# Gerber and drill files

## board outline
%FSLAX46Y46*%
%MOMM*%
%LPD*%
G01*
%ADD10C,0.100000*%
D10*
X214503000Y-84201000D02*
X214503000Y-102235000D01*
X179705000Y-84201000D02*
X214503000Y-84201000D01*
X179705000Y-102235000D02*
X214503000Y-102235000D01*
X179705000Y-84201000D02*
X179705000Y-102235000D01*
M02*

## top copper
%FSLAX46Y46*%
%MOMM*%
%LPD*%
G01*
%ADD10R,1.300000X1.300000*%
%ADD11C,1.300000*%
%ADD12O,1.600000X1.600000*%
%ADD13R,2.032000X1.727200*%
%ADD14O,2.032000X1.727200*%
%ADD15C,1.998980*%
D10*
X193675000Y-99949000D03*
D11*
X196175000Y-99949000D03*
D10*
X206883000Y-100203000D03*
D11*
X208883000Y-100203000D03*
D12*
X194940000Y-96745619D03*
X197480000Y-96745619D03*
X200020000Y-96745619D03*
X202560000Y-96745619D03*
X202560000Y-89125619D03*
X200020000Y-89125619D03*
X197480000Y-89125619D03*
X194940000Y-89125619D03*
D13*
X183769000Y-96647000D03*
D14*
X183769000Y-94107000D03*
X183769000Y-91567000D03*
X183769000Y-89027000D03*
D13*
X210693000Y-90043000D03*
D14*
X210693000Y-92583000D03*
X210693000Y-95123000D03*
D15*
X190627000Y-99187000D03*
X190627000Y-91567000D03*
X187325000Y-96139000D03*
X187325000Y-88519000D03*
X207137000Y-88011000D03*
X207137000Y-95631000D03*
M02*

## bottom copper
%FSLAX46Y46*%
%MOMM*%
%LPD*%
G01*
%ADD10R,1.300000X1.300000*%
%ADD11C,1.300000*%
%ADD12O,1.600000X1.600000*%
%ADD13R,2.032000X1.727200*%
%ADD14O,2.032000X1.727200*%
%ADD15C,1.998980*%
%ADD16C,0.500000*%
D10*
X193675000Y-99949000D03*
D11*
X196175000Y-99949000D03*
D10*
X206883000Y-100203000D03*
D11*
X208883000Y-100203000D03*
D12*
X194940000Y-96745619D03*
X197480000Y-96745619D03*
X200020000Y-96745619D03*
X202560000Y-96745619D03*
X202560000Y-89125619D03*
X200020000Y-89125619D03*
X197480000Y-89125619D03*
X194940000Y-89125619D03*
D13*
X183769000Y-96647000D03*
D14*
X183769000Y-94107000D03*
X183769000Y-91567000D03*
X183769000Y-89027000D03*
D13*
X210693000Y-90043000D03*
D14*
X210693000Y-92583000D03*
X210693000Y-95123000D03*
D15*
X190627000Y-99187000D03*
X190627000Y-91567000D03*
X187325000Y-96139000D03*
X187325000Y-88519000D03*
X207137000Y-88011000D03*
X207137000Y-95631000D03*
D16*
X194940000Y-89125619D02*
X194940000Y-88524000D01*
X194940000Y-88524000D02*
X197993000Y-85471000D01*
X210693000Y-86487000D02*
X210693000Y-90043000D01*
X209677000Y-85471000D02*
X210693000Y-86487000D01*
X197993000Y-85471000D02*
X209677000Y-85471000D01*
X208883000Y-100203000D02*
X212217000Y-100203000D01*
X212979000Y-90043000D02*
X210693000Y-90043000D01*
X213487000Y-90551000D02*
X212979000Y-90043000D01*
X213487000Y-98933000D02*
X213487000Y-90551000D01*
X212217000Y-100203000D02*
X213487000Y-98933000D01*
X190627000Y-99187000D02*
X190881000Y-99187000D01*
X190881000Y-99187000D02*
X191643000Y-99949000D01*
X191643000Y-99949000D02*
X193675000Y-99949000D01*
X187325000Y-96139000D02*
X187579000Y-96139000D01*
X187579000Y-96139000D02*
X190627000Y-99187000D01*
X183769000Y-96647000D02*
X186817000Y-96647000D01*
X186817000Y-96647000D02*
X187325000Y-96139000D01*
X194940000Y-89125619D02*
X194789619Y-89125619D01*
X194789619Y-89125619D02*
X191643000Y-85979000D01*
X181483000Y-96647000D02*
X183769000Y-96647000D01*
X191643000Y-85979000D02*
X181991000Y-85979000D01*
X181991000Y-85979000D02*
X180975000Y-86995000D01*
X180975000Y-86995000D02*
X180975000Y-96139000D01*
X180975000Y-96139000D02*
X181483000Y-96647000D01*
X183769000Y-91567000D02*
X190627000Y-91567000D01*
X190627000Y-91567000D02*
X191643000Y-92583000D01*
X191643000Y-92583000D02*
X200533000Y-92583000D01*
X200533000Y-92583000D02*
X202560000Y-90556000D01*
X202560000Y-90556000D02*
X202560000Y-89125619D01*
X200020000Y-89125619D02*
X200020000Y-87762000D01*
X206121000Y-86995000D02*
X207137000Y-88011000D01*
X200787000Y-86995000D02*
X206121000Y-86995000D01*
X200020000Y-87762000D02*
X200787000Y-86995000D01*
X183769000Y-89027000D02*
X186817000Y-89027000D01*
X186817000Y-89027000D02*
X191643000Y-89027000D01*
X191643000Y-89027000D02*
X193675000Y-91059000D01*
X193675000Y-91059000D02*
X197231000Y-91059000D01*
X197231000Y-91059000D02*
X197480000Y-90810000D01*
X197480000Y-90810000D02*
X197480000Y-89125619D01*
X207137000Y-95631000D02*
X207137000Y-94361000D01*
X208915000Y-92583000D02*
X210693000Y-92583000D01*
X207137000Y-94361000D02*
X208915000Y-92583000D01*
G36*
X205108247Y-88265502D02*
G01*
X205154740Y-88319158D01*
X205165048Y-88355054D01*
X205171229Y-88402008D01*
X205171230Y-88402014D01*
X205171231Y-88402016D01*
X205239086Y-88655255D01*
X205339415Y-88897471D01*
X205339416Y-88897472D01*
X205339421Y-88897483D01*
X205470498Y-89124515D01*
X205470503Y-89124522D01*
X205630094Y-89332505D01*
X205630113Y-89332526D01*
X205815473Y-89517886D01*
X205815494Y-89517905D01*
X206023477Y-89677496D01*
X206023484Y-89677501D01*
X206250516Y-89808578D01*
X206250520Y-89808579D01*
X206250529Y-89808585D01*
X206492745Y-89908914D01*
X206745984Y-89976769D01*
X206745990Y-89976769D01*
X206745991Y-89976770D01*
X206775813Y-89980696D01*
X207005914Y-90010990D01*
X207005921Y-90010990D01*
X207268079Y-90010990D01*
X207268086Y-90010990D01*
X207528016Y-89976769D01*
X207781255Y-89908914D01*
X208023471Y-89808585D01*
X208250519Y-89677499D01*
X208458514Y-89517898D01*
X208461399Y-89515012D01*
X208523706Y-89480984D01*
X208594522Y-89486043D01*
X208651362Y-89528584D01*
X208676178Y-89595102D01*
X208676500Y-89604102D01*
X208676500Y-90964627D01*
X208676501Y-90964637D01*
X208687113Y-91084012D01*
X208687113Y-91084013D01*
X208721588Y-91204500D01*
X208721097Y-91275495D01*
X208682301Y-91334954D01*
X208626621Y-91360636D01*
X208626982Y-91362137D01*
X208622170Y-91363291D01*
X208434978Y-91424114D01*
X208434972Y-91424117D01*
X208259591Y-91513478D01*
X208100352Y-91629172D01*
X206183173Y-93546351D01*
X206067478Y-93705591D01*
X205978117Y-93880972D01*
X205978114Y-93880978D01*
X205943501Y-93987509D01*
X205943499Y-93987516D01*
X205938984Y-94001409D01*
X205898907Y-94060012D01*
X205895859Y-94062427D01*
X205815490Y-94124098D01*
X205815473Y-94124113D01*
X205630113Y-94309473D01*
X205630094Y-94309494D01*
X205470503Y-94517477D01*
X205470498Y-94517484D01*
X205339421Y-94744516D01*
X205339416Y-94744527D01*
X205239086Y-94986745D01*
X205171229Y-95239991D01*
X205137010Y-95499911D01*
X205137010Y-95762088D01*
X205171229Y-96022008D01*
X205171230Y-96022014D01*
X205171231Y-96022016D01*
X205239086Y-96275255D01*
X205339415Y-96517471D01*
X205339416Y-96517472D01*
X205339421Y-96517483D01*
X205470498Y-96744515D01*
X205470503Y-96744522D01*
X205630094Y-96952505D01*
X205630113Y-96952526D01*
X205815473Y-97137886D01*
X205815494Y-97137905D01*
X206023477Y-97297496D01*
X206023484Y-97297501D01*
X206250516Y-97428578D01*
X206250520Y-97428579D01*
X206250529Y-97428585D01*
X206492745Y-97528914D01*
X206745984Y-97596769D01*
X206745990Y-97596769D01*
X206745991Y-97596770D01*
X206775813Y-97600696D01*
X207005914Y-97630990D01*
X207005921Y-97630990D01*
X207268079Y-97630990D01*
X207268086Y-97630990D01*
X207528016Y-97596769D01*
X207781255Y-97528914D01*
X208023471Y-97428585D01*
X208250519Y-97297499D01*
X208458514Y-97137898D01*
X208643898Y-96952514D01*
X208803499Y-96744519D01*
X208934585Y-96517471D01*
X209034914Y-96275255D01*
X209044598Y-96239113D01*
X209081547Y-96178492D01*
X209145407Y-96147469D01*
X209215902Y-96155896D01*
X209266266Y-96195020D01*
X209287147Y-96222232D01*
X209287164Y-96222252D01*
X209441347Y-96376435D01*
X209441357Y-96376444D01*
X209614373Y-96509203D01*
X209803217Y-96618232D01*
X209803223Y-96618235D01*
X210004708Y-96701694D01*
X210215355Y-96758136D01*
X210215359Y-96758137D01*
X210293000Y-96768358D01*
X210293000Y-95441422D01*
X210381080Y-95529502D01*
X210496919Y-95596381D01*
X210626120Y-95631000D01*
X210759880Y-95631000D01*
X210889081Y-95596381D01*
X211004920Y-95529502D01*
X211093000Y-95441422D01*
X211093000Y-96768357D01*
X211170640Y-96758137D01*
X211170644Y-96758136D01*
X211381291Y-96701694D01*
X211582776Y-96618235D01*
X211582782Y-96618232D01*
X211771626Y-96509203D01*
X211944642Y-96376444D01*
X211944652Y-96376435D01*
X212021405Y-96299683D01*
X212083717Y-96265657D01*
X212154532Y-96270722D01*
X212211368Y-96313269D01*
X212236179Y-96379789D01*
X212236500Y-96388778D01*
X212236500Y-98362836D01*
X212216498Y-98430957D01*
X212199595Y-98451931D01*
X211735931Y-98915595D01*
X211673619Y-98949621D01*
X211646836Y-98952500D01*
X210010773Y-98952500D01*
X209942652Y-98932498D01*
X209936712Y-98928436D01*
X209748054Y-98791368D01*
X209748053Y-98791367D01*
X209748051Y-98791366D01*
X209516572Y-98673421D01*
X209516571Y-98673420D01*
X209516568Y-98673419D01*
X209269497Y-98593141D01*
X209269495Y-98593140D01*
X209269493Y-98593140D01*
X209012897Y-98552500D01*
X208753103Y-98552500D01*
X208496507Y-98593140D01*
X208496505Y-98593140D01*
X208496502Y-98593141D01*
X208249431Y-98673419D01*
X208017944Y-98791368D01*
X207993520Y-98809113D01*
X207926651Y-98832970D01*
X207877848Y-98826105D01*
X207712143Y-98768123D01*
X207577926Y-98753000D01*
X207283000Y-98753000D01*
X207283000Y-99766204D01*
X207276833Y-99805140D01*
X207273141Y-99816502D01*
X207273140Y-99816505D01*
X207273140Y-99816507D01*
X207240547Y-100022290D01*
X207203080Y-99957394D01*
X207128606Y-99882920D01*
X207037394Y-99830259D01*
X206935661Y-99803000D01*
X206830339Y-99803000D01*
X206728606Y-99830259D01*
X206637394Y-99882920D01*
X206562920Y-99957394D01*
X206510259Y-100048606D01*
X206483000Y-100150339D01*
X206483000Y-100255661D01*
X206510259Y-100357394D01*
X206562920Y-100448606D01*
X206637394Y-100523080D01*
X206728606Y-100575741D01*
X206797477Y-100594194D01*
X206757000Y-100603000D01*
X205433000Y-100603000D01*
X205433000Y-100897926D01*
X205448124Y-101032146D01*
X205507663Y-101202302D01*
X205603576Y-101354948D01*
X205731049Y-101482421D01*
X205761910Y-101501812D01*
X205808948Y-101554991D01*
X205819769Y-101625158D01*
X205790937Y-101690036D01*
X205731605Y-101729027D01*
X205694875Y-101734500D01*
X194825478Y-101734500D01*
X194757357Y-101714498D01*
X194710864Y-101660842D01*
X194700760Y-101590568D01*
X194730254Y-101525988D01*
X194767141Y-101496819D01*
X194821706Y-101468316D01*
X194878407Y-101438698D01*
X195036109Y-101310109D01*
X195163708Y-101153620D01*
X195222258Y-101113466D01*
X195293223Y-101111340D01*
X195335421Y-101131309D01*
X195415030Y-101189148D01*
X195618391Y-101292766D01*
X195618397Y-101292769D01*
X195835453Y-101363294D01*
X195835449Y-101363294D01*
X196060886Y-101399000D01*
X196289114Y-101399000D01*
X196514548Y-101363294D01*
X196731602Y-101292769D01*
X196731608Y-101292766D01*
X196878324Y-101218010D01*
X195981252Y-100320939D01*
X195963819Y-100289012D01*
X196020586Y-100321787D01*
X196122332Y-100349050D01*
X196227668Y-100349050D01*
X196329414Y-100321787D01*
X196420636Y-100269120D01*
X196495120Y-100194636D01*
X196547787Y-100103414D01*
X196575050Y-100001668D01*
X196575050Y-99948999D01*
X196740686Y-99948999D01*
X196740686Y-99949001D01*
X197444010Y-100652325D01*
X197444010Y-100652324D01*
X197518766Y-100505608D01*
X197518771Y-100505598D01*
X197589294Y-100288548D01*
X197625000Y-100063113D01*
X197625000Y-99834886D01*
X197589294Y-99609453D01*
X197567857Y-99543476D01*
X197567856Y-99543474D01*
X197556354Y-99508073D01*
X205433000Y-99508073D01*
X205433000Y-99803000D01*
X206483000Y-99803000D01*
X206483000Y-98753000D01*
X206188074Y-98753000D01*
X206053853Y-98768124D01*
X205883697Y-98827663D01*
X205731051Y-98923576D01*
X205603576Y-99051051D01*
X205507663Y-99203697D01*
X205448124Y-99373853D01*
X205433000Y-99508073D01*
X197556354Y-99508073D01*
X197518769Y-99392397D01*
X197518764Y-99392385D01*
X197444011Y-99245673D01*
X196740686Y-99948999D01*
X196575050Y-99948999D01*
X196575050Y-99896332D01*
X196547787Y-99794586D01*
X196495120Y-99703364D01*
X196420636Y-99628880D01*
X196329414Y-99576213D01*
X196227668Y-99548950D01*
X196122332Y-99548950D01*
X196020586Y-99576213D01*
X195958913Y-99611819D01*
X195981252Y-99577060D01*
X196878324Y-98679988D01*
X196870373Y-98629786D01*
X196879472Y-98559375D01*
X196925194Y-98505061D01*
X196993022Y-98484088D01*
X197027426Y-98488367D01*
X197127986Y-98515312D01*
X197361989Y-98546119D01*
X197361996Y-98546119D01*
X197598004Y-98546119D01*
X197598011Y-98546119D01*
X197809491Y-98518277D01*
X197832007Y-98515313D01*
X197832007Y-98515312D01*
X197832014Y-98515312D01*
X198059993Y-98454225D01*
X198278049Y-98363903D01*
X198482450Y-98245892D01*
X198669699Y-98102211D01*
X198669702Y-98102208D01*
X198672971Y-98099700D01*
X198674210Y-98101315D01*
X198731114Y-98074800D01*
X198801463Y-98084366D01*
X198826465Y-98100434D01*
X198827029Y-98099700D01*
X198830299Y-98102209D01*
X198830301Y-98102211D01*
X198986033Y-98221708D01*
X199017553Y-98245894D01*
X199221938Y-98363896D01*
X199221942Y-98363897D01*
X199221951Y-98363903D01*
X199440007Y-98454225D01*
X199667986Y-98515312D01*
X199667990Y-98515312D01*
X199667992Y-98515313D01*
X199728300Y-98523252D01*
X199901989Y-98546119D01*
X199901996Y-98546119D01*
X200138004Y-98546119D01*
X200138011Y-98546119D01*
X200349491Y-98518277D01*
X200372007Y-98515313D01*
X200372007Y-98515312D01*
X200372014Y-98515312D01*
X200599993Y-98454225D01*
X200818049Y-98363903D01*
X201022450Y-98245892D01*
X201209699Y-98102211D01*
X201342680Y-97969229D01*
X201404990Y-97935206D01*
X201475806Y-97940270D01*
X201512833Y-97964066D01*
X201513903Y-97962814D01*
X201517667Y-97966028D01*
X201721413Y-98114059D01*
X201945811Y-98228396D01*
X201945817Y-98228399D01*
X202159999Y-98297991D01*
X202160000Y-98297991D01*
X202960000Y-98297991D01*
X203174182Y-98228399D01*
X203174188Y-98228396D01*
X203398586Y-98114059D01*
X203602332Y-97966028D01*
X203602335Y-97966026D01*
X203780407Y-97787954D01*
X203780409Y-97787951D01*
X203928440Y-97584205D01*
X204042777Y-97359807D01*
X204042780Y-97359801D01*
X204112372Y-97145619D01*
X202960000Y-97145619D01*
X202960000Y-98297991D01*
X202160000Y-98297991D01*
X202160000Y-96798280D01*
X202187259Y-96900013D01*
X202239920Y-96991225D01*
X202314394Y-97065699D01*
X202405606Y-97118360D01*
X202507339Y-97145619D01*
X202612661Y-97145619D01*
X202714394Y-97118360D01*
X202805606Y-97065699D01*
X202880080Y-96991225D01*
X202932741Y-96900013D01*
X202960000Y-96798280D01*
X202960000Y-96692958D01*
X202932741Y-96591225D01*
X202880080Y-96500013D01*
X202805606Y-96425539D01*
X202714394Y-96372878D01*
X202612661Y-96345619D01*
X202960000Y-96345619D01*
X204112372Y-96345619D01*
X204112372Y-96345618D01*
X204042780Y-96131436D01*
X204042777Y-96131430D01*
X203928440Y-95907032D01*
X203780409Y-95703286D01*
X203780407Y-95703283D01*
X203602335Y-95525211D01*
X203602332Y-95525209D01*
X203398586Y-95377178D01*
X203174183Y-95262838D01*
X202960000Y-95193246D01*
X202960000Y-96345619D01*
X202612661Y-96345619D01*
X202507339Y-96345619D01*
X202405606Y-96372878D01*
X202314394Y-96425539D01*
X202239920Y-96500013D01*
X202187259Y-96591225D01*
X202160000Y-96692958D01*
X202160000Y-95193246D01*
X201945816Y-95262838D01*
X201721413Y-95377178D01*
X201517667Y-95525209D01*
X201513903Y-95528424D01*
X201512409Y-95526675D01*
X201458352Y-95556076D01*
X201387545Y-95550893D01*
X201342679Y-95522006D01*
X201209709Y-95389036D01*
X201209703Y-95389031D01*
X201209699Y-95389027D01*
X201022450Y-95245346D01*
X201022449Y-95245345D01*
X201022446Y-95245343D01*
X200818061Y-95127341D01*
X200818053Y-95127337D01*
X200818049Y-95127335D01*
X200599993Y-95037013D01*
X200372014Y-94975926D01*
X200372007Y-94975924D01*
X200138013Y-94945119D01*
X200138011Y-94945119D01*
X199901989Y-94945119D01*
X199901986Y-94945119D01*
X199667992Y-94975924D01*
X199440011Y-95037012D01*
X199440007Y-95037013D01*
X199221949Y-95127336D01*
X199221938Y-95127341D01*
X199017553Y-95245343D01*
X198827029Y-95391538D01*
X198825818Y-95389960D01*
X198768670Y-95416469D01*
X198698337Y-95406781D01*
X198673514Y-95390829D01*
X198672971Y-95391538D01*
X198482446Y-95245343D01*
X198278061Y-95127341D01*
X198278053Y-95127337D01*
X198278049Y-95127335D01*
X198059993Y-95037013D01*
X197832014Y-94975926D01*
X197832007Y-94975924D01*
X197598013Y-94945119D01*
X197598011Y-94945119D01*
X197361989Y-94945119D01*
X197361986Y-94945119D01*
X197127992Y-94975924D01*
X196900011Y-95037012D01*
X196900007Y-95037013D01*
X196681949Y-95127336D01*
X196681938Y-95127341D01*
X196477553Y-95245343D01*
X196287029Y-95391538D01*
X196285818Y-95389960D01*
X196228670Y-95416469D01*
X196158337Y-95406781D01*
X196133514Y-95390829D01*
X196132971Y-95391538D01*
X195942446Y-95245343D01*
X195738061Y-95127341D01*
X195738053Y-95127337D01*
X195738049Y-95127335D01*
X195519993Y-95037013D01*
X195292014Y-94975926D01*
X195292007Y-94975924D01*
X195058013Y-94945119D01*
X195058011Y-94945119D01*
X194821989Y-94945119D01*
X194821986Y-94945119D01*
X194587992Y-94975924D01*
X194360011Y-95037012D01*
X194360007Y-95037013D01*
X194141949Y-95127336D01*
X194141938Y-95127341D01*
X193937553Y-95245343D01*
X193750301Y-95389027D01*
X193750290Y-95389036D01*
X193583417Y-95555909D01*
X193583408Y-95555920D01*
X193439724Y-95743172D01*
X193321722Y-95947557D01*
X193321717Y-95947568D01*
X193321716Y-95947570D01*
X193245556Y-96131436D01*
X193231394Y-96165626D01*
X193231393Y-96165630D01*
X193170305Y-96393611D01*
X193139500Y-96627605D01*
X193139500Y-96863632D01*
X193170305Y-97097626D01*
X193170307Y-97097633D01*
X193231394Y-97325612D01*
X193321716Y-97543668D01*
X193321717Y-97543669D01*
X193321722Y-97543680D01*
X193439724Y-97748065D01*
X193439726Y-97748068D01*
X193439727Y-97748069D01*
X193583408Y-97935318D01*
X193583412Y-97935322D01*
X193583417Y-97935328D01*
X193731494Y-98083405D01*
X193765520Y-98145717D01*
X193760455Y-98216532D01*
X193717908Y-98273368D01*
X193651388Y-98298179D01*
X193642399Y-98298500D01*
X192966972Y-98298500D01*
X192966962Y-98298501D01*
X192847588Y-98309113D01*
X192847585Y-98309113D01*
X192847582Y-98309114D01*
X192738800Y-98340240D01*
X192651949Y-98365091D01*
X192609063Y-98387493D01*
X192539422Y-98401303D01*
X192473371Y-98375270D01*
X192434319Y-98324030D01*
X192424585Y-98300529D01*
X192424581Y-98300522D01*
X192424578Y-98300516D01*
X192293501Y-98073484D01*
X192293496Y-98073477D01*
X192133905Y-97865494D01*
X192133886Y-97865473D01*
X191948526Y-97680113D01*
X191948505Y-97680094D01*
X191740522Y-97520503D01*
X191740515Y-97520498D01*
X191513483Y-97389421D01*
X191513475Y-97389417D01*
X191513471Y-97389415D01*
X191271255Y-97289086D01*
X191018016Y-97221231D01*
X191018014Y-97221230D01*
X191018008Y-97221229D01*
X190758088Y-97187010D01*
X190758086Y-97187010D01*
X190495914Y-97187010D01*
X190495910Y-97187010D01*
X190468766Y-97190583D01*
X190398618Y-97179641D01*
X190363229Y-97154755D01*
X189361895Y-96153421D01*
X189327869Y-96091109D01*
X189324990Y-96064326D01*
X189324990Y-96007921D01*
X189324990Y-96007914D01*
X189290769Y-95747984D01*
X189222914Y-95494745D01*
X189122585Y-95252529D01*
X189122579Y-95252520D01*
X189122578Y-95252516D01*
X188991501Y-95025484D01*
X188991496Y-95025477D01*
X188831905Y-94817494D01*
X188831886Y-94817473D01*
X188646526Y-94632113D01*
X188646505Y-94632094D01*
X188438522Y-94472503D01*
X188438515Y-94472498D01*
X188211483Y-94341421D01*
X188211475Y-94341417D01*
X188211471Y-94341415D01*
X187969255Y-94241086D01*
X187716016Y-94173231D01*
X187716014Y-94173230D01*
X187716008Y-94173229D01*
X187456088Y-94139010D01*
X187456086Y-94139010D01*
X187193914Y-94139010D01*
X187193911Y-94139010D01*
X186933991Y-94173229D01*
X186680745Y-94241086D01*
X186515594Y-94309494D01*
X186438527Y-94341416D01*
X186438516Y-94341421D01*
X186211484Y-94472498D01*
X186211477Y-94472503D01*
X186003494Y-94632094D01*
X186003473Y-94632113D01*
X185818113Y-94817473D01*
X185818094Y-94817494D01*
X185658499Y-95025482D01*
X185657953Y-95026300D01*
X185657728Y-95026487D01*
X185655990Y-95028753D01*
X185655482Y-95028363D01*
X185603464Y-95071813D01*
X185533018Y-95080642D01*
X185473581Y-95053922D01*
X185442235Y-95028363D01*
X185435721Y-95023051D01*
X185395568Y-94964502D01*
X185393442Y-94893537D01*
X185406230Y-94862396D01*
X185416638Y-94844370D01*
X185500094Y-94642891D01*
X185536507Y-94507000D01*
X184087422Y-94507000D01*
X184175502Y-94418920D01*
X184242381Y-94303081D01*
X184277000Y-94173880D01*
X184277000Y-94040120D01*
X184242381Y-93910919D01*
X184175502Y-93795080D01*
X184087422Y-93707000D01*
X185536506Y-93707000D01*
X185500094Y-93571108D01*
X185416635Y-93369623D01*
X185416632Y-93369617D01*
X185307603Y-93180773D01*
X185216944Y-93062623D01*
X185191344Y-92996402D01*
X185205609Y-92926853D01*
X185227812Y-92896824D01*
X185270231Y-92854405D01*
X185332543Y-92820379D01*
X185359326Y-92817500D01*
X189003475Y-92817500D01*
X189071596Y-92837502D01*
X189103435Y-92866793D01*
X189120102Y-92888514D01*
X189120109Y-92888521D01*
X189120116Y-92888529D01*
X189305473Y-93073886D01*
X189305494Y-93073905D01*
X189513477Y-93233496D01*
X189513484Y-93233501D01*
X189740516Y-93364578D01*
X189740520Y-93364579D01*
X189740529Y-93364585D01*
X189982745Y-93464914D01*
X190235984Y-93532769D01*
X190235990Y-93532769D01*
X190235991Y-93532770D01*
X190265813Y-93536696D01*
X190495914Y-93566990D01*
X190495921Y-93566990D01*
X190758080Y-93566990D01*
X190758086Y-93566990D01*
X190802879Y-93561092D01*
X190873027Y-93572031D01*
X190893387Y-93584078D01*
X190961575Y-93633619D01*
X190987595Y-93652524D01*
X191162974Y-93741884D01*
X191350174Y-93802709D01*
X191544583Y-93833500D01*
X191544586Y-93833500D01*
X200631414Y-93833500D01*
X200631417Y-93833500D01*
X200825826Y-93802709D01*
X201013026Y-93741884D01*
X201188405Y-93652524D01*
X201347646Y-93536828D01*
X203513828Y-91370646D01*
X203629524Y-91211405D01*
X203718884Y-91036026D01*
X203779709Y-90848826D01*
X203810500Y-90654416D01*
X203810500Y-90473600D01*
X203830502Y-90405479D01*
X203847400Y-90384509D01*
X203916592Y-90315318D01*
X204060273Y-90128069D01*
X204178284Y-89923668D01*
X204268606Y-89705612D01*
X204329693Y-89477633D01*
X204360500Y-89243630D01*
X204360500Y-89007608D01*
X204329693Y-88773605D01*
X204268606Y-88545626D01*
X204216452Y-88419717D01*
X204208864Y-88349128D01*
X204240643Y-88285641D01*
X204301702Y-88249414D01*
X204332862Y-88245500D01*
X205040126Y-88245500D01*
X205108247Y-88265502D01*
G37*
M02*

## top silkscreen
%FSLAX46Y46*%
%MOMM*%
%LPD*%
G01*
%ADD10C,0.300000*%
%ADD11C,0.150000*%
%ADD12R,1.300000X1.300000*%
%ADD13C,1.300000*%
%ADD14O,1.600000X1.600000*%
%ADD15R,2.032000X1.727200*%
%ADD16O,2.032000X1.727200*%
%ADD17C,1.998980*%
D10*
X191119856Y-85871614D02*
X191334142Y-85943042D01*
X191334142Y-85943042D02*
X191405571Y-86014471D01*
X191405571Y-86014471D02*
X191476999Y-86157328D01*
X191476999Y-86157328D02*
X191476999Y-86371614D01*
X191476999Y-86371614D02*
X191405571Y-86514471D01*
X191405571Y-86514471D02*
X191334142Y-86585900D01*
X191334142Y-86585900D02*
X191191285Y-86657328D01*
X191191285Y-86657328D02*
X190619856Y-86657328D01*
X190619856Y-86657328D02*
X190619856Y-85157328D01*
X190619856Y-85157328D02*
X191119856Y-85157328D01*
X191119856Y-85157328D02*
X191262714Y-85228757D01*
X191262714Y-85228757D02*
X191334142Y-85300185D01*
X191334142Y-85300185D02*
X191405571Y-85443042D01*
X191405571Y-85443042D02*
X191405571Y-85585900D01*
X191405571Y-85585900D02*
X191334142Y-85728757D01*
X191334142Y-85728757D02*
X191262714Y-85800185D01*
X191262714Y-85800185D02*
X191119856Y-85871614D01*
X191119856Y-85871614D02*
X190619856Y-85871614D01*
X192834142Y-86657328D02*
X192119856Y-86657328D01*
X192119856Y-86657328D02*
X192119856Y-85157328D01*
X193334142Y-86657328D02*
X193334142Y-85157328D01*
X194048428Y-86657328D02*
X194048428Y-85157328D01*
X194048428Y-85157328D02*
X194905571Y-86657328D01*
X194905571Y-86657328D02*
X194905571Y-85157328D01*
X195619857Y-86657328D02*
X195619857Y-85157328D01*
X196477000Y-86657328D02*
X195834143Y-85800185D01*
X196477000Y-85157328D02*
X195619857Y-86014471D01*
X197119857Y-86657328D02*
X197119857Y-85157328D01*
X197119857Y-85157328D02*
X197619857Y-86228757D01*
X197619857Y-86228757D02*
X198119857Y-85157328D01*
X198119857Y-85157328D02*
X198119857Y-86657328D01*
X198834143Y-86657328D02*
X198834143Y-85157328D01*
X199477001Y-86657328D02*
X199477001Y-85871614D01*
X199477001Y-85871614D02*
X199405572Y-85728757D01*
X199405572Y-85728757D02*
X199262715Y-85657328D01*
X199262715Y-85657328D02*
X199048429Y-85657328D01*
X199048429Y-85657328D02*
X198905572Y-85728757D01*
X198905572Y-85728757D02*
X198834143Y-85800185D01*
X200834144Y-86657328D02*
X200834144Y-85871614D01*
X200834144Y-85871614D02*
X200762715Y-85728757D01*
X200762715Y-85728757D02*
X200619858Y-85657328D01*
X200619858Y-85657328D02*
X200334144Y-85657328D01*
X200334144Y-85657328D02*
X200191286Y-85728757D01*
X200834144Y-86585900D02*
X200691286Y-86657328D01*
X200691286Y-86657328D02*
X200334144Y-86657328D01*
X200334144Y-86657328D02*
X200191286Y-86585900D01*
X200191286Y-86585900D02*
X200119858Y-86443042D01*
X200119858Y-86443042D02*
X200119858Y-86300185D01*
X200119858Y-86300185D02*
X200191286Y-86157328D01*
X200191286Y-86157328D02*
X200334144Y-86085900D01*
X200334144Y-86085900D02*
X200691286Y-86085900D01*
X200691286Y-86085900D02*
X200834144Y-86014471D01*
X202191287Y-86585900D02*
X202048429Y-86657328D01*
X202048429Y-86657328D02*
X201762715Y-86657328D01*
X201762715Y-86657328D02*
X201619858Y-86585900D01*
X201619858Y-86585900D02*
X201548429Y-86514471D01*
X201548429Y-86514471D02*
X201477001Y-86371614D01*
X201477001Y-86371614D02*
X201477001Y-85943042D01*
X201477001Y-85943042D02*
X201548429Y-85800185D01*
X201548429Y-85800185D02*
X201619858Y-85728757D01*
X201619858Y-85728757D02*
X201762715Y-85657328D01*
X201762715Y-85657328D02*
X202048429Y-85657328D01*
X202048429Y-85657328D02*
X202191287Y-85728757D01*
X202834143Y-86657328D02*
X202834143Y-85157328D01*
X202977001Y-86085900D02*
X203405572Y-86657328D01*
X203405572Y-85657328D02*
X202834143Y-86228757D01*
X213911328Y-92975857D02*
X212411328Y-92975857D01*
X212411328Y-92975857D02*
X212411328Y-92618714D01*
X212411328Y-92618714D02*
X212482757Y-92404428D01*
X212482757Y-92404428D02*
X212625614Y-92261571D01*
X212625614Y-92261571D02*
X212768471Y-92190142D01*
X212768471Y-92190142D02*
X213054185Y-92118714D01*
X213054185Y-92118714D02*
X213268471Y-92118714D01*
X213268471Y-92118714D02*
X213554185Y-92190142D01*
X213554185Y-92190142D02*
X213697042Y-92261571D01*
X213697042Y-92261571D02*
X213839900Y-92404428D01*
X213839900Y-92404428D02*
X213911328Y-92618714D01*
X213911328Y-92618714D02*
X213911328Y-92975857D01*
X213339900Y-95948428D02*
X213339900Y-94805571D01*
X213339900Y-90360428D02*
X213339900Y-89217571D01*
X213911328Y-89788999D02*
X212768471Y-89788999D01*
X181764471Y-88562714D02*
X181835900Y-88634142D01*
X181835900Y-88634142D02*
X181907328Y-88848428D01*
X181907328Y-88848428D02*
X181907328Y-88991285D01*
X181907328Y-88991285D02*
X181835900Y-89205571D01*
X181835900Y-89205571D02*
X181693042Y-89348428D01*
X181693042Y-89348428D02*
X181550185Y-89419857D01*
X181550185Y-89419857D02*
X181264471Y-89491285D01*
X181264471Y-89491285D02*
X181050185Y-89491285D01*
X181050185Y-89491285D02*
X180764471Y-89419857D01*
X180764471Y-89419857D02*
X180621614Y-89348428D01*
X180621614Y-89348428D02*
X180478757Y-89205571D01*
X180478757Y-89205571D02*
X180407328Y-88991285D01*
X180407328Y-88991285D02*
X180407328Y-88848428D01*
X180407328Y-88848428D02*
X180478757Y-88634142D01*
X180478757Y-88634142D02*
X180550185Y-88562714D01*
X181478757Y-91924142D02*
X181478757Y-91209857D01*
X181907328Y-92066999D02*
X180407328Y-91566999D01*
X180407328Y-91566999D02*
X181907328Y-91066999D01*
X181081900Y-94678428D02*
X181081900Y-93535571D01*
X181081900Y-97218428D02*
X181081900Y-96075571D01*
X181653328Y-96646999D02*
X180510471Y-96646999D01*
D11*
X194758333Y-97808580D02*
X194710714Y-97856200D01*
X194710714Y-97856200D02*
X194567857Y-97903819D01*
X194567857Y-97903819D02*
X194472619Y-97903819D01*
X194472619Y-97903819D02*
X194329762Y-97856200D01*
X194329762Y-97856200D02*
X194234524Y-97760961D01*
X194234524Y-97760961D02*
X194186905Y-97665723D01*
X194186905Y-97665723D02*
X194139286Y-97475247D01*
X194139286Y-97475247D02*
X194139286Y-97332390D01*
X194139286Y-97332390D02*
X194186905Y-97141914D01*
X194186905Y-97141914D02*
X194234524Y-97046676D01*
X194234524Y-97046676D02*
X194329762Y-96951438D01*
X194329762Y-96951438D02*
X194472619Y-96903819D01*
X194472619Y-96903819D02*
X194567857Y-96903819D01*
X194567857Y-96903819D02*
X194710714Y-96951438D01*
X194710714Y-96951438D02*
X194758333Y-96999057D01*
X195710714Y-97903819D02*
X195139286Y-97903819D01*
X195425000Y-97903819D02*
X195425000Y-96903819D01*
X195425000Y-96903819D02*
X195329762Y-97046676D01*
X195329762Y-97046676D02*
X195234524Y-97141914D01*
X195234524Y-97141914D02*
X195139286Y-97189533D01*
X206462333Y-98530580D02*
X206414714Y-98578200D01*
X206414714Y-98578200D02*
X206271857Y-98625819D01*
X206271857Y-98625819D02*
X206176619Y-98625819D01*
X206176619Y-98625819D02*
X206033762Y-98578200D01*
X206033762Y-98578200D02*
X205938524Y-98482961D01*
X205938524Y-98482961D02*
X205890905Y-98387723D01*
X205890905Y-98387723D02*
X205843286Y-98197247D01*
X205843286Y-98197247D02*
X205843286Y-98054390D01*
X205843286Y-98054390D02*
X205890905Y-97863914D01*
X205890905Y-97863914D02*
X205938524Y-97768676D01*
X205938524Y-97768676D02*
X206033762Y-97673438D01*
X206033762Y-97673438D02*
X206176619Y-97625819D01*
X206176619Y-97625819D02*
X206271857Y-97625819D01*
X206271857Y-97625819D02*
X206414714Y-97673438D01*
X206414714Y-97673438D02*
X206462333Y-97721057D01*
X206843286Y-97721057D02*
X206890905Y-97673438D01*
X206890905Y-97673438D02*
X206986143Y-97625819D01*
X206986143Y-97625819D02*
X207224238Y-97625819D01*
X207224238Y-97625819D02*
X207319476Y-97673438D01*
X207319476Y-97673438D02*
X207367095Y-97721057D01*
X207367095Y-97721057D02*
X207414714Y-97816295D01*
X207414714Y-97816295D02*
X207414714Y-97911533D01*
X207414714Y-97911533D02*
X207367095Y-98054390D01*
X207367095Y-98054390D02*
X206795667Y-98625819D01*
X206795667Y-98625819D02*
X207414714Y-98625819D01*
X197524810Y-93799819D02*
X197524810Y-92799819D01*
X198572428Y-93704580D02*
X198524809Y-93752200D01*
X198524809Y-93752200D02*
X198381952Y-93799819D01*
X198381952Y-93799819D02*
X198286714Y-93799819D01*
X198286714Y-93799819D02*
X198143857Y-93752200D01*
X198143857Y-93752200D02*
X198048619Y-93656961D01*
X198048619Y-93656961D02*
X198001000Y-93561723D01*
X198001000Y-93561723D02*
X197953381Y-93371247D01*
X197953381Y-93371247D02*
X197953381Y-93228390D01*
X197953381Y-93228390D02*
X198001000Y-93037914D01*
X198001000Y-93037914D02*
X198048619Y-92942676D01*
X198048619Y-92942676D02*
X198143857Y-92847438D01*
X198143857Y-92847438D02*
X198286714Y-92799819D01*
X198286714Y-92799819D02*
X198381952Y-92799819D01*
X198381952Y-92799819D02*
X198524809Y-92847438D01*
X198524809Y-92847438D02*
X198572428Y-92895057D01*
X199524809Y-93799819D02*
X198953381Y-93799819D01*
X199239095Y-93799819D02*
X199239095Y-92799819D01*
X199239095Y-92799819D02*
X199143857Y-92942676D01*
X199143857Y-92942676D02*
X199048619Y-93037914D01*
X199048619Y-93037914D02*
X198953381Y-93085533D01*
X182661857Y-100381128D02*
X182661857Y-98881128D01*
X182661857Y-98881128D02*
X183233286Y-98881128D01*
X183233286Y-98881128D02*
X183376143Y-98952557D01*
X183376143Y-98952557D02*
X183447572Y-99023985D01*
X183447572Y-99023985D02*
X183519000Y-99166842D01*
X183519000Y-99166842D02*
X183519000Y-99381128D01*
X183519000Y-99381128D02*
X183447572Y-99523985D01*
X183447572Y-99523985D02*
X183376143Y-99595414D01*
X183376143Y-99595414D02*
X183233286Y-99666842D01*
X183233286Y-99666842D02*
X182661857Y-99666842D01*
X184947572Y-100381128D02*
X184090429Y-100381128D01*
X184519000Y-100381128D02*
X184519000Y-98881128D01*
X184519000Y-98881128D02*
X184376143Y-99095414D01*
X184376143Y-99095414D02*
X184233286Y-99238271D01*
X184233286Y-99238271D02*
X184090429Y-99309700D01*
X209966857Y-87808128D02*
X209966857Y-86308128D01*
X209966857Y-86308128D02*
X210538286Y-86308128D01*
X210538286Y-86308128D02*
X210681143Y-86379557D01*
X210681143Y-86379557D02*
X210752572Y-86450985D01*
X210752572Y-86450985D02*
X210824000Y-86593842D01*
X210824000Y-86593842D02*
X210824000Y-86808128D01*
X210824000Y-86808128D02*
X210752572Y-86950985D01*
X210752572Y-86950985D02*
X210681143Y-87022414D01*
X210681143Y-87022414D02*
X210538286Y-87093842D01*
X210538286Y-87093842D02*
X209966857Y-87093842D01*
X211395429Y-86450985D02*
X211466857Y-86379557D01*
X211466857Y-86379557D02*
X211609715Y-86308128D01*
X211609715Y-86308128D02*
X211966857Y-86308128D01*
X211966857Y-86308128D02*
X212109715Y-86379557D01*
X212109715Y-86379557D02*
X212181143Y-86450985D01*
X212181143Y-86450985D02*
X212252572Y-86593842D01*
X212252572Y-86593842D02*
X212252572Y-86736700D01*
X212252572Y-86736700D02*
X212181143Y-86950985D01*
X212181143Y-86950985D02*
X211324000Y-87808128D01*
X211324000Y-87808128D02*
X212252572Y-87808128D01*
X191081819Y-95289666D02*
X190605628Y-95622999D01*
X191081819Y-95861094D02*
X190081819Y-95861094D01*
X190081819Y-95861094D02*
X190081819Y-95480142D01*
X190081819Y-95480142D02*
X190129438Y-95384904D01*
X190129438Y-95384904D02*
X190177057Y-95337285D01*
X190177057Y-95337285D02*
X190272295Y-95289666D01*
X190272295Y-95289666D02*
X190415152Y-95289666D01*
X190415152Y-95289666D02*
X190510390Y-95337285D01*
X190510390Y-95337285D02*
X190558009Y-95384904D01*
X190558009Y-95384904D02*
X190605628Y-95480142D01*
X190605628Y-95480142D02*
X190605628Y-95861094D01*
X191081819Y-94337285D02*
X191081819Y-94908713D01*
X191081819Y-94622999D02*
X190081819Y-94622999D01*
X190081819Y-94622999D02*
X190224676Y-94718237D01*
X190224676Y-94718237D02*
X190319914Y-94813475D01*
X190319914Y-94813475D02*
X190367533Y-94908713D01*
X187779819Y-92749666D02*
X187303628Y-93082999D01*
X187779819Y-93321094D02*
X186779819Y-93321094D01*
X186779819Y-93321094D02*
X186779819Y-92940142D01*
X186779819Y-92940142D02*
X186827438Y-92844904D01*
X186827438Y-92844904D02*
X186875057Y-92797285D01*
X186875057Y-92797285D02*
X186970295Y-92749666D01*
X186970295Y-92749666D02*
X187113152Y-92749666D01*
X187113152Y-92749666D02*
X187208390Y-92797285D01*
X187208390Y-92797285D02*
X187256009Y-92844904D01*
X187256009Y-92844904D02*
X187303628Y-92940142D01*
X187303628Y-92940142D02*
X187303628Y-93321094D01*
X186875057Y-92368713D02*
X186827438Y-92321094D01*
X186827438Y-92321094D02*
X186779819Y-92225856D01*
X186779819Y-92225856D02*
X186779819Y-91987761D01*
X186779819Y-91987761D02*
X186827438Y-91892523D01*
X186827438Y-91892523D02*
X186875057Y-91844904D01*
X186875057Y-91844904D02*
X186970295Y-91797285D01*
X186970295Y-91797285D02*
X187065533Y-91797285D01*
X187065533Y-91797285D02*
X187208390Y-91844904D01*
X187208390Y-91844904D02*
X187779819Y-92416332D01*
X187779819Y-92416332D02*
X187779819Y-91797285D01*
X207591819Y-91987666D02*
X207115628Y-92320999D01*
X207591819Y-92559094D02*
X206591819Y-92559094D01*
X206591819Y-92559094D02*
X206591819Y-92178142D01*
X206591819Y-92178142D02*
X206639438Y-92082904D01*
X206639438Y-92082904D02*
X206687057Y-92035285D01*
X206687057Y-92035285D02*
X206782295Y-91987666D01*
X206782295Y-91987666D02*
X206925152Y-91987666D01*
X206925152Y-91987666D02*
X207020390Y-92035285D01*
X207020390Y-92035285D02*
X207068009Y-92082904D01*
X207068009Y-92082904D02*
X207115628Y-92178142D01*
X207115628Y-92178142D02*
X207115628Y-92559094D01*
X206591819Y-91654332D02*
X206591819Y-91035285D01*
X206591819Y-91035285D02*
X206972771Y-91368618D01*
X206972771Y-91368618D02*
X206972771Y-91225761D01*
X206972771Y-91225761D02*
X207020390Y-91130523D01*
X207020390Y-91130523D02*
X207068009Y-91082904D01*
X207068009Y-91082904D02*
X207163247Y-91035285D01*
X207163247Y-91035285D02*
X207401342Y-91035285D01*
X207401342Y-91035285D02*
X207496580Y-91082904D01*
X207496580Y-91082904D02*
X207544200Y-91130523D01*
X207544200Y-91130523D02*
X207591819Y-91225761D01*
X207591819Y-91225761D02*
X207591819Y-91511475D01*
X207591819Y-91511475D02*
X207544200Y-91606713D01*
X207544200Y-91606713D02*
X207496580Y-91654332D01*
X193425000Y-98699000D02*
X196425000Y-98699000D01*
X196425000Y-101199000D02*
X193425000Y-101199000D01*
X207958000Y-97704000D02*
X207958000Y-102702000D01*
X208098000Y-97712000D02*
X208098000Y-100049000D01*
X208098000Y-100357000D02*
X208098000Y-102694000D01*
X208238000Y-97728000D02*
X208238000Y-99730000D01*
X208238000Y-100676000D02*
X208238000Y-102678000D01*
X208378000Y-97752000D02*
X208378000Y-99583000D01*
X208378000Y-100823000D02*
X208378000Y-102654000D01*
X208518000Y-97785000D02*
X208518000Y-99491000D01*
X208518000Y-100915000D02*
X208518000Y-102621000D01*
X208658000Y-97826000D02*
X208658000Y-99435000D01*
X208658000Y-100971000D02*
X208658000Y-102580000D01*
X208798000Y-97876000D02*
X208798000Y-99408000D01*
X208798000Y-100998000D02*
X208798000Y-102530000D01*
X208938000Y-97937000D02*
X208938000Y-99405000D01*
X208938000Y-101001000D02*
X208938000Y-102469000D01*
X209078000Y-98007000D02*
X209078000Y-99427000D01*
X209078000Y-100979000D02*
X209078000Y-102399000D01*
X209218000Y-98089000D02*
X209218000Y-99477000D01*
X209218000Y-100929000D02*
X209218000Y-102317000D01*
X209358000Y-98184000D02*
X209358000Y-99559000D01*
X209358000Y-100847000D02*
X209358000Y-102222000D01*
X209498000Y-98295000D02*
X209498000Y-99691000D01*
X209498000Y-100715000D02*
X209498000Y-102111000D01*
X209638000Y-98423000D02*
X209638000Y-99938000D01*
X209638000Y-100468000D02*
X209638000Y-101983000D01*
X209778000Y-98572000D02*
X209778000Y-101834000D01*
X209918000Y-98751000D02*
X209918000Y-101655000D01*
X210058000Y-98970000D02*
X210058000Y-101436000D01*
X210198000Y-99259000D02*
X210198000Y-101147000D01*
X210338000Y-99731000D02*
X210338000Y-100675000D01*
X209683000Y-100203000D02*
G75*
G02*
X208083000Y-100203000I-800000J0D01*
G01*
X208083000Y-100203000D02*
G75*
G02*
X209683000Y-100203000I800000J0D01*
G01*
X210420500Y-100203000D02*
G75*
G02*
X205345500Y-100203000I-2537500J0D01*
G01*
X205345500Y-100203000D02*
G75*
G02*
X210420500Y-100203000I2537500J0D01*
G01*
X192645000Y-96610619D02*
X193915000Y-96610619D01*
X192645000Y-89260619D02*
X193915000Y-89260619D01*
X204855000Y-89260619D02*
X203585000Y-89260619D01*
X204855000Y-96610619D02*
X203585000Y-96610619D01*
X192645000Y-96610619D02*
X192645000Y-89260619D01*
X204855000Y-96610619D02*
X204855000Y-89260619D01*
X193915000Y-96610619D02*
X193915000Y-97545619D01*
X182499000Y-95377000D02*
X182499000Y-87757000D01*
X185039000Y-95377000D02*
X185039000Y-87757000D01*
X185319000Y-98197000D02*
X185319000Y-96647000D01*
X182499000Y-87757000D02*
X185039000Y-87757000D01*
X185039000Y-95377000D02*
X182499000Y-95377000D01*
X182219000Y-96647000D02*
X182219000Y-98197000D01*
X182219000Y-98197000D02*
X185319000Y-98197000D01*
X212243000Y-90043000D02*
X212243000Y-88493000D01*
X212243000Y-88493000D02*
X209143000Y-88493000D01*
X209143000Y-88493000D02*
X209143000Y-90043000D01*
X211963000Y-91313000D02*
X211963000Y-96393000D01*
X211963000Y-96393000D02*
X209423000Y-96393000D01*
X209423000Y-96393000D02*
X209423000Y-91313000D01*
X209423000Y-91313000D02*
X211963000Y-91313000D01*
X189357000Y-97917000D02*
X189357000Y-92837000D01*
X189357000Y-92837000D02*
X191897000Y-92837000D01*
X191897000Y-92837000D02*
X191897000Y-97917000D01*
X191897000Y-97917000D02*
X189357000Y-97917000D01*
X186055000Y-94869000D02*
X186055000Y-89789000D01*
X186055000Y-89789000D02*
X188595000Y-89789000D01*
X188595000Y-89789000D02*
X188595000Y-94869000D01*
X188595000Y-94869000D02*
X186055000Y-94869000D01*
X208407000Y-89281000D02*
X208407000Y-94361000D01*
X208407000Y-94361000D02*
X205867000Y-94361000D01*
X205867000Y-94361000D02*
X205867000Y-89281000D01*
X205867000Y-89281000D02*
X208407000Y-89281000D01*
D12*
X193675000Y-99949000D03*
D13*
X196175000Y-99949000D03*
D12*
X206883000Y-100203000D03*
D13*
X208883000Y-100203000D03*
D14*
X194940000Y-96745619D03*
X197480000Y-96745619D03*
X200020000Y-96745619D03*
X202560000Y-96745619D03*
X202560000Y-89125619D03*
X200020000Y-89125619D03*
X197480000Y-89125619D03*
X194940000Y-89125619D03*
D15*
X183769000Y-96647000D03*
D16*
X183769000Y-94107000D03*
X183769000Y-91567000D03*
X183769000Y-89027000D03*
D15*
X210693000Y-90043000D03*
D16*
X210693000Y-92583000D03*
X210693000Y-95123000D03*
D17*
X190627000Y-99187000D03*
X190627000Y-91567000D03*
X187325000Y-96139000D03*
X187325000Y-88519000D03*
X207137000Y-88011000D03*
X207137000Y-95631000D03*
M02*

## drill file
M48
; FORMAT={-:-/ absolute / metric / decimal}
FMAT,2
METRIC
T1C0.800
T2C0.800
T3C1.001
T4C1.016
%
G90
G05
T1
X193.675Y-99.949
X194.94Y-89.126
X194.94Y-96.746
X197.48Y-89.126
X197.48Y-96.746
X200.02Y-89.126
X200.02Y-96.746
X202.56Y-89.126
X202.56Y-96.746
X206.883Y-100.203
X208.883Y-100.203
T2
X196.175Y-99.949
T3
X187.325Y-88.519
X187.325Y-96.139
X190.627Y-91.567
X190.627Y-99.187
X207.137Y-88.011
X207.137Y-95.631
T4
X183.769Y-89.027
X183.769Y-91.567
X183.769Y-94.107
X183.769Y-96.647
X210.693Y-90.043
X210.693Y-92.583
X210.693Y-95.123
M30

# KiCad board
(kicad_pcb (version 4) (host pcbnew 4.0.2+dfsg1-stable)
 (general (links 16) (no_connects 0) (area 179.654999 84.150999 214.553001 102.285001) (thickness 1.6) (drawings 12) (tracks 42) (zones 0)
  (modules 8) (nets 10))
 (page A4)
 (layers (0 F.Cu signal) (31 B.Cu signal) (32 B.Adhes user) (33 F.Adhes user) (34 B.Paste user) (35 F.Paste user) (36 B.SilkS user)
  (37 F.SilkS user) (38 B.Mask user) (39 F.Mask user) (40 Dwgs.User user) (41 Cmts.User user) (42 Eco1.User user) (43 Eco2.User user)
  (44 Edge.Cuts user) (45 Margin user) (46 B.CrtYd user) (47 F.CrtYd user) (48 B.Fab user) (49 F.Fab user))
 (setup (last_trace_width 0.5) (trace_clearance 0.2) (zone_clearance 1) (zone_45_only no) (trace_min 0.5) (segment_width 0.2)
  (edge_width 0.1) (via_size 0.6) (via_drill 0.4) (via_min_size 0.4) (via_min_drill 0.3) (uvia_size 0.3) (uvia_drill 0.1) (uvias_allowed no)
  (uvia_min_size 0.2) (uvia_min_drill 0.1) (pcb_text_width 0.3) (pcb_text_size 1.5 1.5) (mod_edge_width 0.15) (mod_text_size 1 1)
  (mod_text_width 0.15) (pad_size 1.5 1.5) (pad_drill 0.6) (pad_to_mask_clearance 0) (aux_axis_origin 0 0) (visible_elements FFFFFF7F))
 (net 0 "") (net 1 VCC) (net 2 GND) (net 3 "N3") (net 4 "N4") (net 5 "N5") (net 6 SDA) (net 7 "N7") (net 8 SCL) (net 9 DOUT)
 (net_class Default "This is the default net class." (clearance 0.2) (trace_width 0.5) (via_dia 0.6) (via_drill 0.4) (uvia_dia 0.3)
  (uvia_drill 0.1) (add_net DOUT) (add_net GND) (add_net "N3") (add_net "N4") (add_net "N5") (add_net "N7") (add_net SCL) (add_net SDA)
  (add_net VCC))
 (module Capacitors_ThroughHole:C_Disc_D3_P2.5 (layer F.Cu) (at 193.675 99.949)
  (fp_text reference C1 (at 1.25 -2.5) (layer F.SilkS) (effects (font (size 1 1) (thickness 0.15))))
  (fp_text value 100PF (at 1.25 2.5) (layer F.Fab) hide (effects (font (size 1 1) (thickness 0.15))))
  (fp_line (start -0.25 -1.25) (end 2.75 -1.25) (layer F.SilkS) (width 0.15))
  (fp_line (start 2.75 1.25) (end -0.25 1.25) (layer F.SilkS) (width 0.15))
  (pad 1 thru_hole rect (at 0 0) (size 1.3 1.3) (drill 0.8) (layers *.Cu *.Mask F.SilkS) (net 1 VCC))
  (pad 2 thru_hole circle (at 2.5 0) (size 1.3 1.3) (drill 0.8001) (layers *.Cu *.Mask F.SilkS) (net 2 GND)))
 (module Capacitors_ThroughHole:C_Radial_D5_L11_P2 (layer F.Cu) (at 206.883 100.203)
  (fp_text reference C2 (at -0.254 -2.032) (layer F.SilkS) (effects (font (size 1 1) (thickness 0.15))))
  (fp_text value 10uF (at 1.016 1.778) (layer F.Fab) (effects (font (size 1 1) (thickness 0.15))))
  (fp_line (start 1.075 -2.499) (end 1.075 2.499) (layer F.SilkS) (width 0.15))
  (fp_line (start 1.215 -2.491) (end 1.215 -0.154) (layer F.SilkS) (width 0.15))
  (fp_line (start 1.215 0.154) (end 1.215 2.491) (layer F.SilkS) (width 0.15))
  (fp_line (start 1.355 -2.475) (end 1.355 -0.473) (layer F.SilkS) (width 0.15))
  (fp_line (start 1.355 0.473) (end 1.355 2.475) (layer F.SilkS) (width 0.15))
  (fp_line (start 1.495 -2.451) (end 1.495 -0.62) (layer F.SilkS) (width 0.15))
  (fp_line (start 1.495 0.62) (end 1.495 2.451) (layer F.SilkS) (width 0.15))
  (fp_line (start 1.635 -2.418) (end 1.635 -0.712) (layer F.SilkS) (width 0.15))
  (fp_line (start 1.635 0.712) (end 1.635 2.418) (layer F.SilkS) (width 0.15))
  (fp_line (start 1.775 -2.377) (end 1.775 -0.768) (layer F.SilkS) (width 0.15))
  (fp_line (start 1.775 0.768) (end 1.775 2.377) (layer F.SilkS) (width 0.15))
  (fp_line (start 1.915 -2.327) (end 1.915 -0.795) (layer F.SilkS) (width 0.15))
  (fp_line (start 1.915 0.795) (end 1.915 2.327) (layer F.SilkS) (width 0.15))
  (fp_line (start 2.055 -2.266) (end 2.055 -0.798) (layer F.SilkS) (width 0.15))
  (fp_line (start 2.055 0.798) (end 2.055 2.266) (layer F.SilkS) (width 0.15))
  (fp_line (start 2.195 -2.196) (end 2.195 -0.776) (layer F.SilkS) (width 0.15))
  (fp_line (start 2.195 0.776) (end 2.195 2.196) (layer F.SilkS) (width 0.15))
  (fp_line (start 2.335 -2.114) (end 2.335 -0.726) (layer F.SilkS) (width 0.15))
  (fp_line (start 2.335 0.726) (end 2.335 2.114) (layer F.SilkS) (width 0.15))
  (fp_line (start 2.475 -2.019) (end 2.475 -0.644) (layer F.SilkS) (width 0.15))
  (fp_line (start 2.475 0.644) (end 2.475 2.019) (layer F.SilkS) (width 0.15))
  (fp_line (start 2.615 -1.908) (end 2.615 -0.512) (layer F.SilkS) (width 0.15))
  (fp_line (start 2.615 0.512) (end 2.615 1.908) (layer F.SilkS) (width 0.15))
  (fp_line (start 2.755 -1.78) (end 2.755 -0.265) (layer F.SilkS) (width 0.15))
  (fp_line (start 2.755 0.265) (end 2.755 1.78) (layer F.SilkS) (width 0.15))
  (fp_line (start 2.895 -1.631) (end 2.895 1.631) (layer F.SilkS) (width 0.15))
  (fp_line (start 3.035 -1.452) (end 3.035 1.452) (layer F.SilkS) (width 0.15))
  (fp_line (start 3.175 -1.233) (end 3.175 1.233) (layer F.SilkS) (width 0.15))
  (fp_line (start 3.315 -0.944) (end 3.315 0.944) (layer F.SilkS) (width 0.15))
  (fp_line (start 3.455 -0.472) (end 3.455 0.472) (layer F.SilkS) (width 0.15))
  (fp_circle (center 2 0) (end 2 -0.8) (layer F.SilkS) (width 0.15))
  (fp_circle (center 1 0) (end 1 -2.5375) (layer F.SilkS) (width 0.15))
  (pad 1 thru_hole rect (at 0 0) (size 1.3 1.3) (drill 0.8) (layers *.Cu *.Mask F.SilkS) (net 2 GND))
  (pad 2 thru_hole circle (at 2 0) (size 1.3 1.3) (drill 0.8) (layers *.Cu *.Mask F.SilkS) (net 1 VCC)))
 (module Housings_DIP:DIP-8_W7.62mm (layer F.Cu) (at 194.94 96.745619 90)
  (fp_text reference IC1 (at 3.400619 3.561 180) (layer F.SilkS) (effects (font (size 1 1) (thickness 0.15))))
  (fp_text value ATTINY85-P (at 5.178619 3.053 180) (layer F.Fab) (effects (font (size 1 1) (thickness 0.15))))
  (fp_line (start 0.135 -2.295) (end 0.135 -1.025) (layer F.SilkS) (width 0.15))
  (fp_line (start 7.485 -2.295) (end 7.485 -1.025) (layer F.SilkS) (width 0.15))
  (fp_line (start 7.485 9.915) (end 7.485 8.645) (layer F.SilkS) (width 0.15))
  (fp_line (start 0.135 9.915) (end 0.135 8.645) (layer F.SilkS) (width 0.15))
  (fp_line (start 0.135 -2.295) (end 7.485 -2.295) (layer F.SilkS) (width 0.15))
  (fp_line (start 0.135 9.915) (end 7.485 9.915) (layer F.SilkS) (width 0.15))
  (fp_line (start 0.135 -1.025) (end -0.8 -1.025) (layer F.SilkS) (width 0.15))
  (pad 1 thru_hole oval (at 0 0 90) (size 1.6 1.6) (drill 0.8) (layers *.Cu *.Mask F.SilkS) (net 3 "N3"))
  (pad 2 thru_hole oval (at 0 2.54 90) (size 1.6 1.6) (drill 0.8) (layers *.Cu *.Mask F.SilkS) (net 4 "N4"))
  (pad 3 thru_hole oval (at 0 5.08 90) (size 1.6 1.6) (drill 0.8) (layers *.Cu *.Mask F.SilkS) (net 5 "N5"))
  (pad 4 thru_hole oval (at 0 7.62 90) (size 1.6 1.6) (drill 0.8) (layers *.Cu *.Mask F.SilkS) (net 2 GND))
  (pad 5 thru_hole oval (at 7.62 7.62 90) (size 1.6 1.6) (drill 0.8) (layers *.Cu *.Mask F.SilkS) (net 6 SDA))
  (pad 6 thru_hole oval (at 7.62 5.08 90) (size 1.6 1.6) (drill 0.8) (layers *.Cu *.Mask F.SilkS) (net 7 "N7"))
  (pad 7 thru_hole oval (at 7.62 2.54 90) (size 1.6 1.6) (drill 0.8) (layers *.Cu *.Mask F.SilkS) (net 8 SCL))
  (pad 8 thru_hole oval (at 7.62 0 90) (size 1.6 1.6) (drill 0.8) (layers *.Cu *.Mask F.SilkS) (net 1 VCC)))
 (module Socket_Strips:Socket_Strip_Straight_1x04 (layer F.Cu) (at 183.769 96.647 90)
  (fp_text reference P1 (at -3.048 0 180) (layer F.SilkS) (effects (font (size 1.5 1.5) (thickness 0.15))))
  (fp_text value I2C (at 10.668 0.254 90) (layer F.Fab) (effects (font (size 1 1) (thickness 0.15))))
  (fp_line (start 1.27 -1.27) (end 8.89 -1.27) (layer F.SilkS) (width 0.15))
  (fp_line (start 1.27 1.27) (end 8.89 1.27) (layer F.SilkS) (width 0.15))
  (fp_line (start -1.55 1.55) (end 0 1.55) (layer F.SilkS) (width 0.15))
  (fp_line (start 8.89 -1.27) (end 8.89 1.27) (layer F.SilkS) (width 0.15))
  (fp_line (start 1.27 1.27) (end 1.27 -1.27) (layer F.SilkS) (width 0.15))
  (fp_line (start 0 -1.55) (end -1.55 -1.55) (layer F.SilkS) (width 0.15))
  (fp_line (start -1.55 -1.55) (end -1.55 1.55) (layer F.SilkS) (width 0.15))
  (pad 1 thru_hole rect (at 0 0 90) (size 1.7272 2.032) (drill 1.016) (layers *.Cu *.Mask F.SilkS) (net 1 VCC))
  (pad 2 thru_hole oval (at 2.54 0 90) (size 1.7272 2.032) (drill 1.016) (layers *.Cu *.Mask F.SilkS) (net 2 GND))
  (pad 3 thru_hole oval (at 5.08 0 90) (size 1.7272 2.032) (drill 1.016) (layers *.Cu *.Mask F.SilkS) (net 6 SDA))
  (pad 4 thru_hole oval (at 7.62 0 90) (size 1.7272 2.032) (drill 1.016) (layers *.Cu *.Mask F.SilkS) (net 8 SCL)))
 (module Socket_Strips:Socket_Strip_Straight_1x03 (layer F.Cu) (at 210.693 90.043 270)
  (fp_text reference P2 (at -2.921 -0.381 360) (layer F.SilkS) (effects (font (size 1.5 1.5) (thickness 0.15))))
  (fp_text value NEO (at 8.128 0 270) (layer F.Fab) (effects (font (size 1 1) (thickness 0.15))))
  (fp_line (start 0 -1.55) (end -1.55 -1.55) (layer F.SilkS) (width 0.15))
  (fp_line (start -1.55 -1.55) (end -1.55 1.55) (layer F.SilkS) (width 0.15))
  (fp_line (start -1.55 1.55) (end 0 1.55) (layer F.SilkS) (width 0.15))
  (fp_line (start 1.27 -1.27) (end 6.35 -1.27) (layer F.SilkS) (width 0.15))
  (fp_line (start 6.35 -1.27) (end 6.35 1.27) (layer F.SilkS) (width 0.15))
  (fp_line (start 6.35 1.27) (end 1.27 1.27) (layer F.SilkS) (width 0.15))
  (fp_line (start 1.27 1.27) (end 1.27 -1.27) (layer F.SilkS) (width 0.15))
  (pad 1 thru_hole rect (at 0 0 270) (size 1.7272 2.032) (drill 1.016) (layers *.Cu *.Mask F.SilkS) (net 1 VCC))
  (pad 2 thru_hole oval (at 2.54 0 270) (size 1.7272 2.032) (drill 1.016) (layers *.Cu *.Mask F.SilkS) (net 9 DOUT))
  (pad 3 thru_hole oval (at 5.08 0 270) (size 1.7272 2.032) (drill 1.016) (layers *.Cu *.Mask F.SilkS) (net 2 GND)))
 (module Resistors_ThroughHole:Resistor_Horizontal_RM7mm (layer F.Cu) (at 190.627 99.187 90)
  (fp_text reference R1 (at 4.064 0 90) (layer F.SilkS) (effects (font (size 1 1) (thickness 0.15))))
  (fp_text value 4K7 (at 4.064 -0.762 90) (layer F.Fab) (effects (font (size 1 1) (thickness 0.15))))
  (fp_line (start 1.27 -1.27) (end 6.35 -1.27) (layer F.SilkS) (width 0.15))
  (fp_line (start 6.35 -1.27) (end 6.35 1.27) (layer F.SilkS) (width 0.15))
  (fp_line (start 6.35 1.27) (end 1.27 1.27) (layer F.SilkS) (width 0.15))
  (fp_line (start 1.27 1.27) (end 1.27 -1.27) (layer F.SilkS) (width 0.15))
  (pad 1 thru_hole circle (at 0 0 90) (size 1.99898 1.99898) (drill 1.00076) (layers *.Cu *.SilkS *.Mask) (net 1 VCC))
  (pad 2 thru_hole circle (at 7.62 0 90) (size 1.99898 1.99898) (drill 1.00076) (layers *.Cu *.SilkS *.Mask) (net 6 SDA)))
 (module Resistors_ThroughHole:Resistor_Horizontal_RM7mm (layer F.Cu) (at 187.325 96.139 90)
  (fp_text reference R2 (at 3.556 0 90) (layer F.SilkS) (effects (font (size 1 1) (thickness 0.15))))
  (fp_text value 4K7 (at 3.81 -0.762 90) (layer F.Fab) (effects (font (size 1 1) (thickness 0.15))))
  (fp_line (start 1.27 -1.27) (end 6.35 -1.27) (layer F.SilkS) (width 0.15))
  (fp_line (start 6.35 -1.27) (end 6.35 1.27) (layer F.SilkS) (width 0.15))
  (fp_line (start 6.35 1.27) (end 1.27 1.27) (layer F.SilkS) (width 0.15))
  (fp_line (start 1.27 1.27) (end 1.27 -1.27) (layer F.SilkS) (width 0.15))
  (pad 1 thru_hole circle (at 0 0 90) (size 1.99898 1.99898) (drill 1.00076) (layers *.Cu *.SilkS *.Mask) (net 1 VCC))
  (pad 2 thru_hole circle (at 7.62 0 90) (size 1.99898 1.99898) (drill 1.00076) (layers *.Cu *.SilkS *.Mask) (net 8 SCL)))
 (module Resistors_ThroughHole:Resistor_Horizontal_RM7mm (layer F.Cu) (at 207.137 88.011 270)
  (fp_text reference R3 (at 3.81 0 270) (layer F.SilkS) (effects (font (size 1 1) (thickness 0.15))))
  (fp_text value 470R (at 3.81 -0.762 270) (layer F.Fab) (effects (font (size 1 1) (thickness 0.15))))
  (fp_line (start 1.27 -1.27) (end 6.35 -1.27) (layer F.SilkS) (width 0.15))
  (fp_line (start 6.35 -1.27) (end 6.35 1.27) (layer F.SilkS) (width 0.15))
  (fp_line (start 6.35 1.27) (end 1.27 1.27) (layer F.SilkS) (width 0.15))
  (fp_line (start 1.27 1.27) (end 1.27 -1.27) (layer F.SilkS) (width 0.15))
  (pad 1 thru_hole circle (at 0 0 270) (size 1.99898 1.99898) (drill 1.00076) (layers *.Cu *.SilkS *.Mask) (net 7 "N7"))
  (pad 2 thru_hole circle (at 7.62 0 270) (size 1.99898 1.99898) (drill 1.00076) (layers *.Cu *.SilkS *.Mask) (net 9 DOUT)))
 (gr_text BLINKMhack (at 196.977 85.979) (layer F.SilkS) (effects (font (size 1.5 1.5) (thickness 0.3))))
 (gr_line (start 214.503 84.201) (end 214.503 102.235) (angle 90) (layer Edge.Cuts) (width 0.1))
 (gr_line (start 179.705 84.201) (end 214.503 84.201) (angle 90) (layer Edge.Cuts) (width 0.1))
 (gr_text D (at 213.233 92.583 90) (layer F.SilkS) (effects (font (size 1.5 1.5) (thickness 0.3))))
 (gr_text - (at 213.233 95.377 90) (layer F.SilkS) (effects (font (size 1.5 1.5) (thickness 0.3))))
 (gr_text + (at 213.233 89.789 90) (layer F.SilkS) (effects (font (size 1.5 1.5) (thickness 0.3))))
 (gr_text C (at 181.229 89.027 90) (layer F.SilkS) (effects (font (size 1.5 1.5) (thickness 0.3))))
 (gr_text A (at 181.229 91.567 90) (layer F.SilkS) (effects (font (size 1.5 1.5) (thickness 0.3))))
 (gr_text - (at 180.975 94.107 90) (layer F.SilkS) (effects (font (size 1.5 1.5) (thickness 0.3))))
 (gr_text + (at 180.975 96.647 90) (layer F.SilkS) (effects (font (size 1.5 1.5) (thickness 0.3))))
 (gr_line (start 179.705 102.235) (end 214.503 102.235) (angle 90) (layer Edge.Cuts) (width 0.1))
 (gr_line (start 179.705 84.201) (end 179.705 102.235) (angle 90) (layer Edge.Cuts) (width 0.1))
 (segment (start 194.94 89.125619) (end 194.94 88.524) (width 0.5) (layer B.Cu) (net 1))
 (segment (start 194.94 88.524) (end 197.993 85.471) (width 0.5) (layer B.Cu) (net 1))
 (segment (start 210.693 86.487) (end 210.693 90.043) (width 0.5) (layer B.Cu) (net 1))
 (segment (start 209.677 85.471) (end 210.693 86.487) (width 0.5) (layer B.Cu) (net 1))
 (segment (start 197.993 85.471) (end 209.677 85.471) (width 0.5) (layer B.Cu) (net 1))
 (segment (start 208.883 100.203) (end 212.217 100.203) (width 0.5) (layer B.Cu) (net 1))
 (segment (start 212.979 90.043) (end 210.693 90.043) (width 0.5) (layer B.Cu) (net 1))
 (segment (start 213.487 90.551) (end 212.979 90.043) (width 0.5) (layer B.Cu) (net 1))
 (segment (start 213.487 98.933) (end 213.487 90.551) (width 0.5) (layer B.Cu) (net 1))
 (segment (start 212.217 100.203) (end 213.487 98.933) (width 0.5) (layer B.Cu) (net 1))
 (segment (start 190.627 99.187) (end 190.881 99.187) (width 0.5) (layer B.Cu) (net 1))
 (segment (start 190.881 99.187) (end 191.643 99.949) (width 0.5) (layer B.Cu) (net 1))
 (segment (start 191.643 99.949) (end 193.675 99.949) (width 0.5) (layer B.Cu) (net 1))
 (segment (start 187.325 96.139) (end 187.579 96.139) (width 0.5) (layer B.Cu) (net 1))
 (segment (start 187.579 96.139) (end 190.627 99.187) (width 0.5) (layer B.Cu) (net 1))
 (segment (start 183.769 96.647) (end 186.817 96.647) (width 0.5) (layer B.Cu) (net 1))
 (segment (start 186.817 96.647) (end 187.325 96.139) (width 0.5) (layer B.Cu) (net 1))
 (segment (start 194.94 89.125619) (end 194.789619 89.125619) (width 0.5) (layer B.Cu) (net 1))
 (segment (start 194.789619 89.125619) (end 191.643 85.979) (width 0.5) (layer B.Cu) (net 1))
 (segment (start 181.483 96.647) (end 183.769 96.647) (width 0.5) (layer B.Cu) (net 1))
 (segment (start 191.643 85.979) (end 181.991 85.979) (width 0.5) (layer B.Cu) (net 1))
 (segment (start 181.991 85.979) (end 180.975 86.995) (width 0.5) (layer B.Cu) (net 1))
 (segment (start 180.975 86.995) (end 180.975 96.139) (width 0.5) (layer B.Cu) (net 1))
 (segment (start 180.975 96.139) (end 181.483 96.647) (width 0.5) (layer B.Cu) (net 1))
 (segment (start 183.769 91.567) (end 190.627 91.567) (width 0.5) (layer B.Cu) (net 6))
 (segment (start 190.627 91.567) (end 191.643 92.583) (width 0.5) (layer B.Cu) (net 6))
 (segment (start 191.643 92.583) (end 200.533 92.583) (width 0.5) (layer B.Cu) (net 6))
 (segment (start 200.533 92.583) (end 202.56 90.556) (width 0.5) (layer B.Cu) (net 6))
 (segment (start 202.56 90.556) (end 202.56 89.125619) (width 0.5) (layer B.Cu) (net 6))
 (segment (start 200.02 89.125619) (end 200.02 87.762) (width 0.5) (layer B.Cu) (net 7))
 (segment (start 206.121 86.995) (end 207.137 88.011) (width 0.5) (layer B.Cu) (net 7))
 (segment (start 200.787 86.995) (end 206.121 86.995) (width 0.5) (layer B.Cu) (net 7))
 (segment (start 200.02 87.762) (end 200.787 86.995) (width 0.5) (layer B.Cu) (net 7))
 (segment (start 183.769 89.027) (end 186.817 89.027) (width 0.5) (layer B.Cu) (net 8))
 (segment (start 186.817 89.027) (end 191.643 89.027) (width 0.5) (layer B.Cu) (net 8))
 (segment (start 191.643 89.027) (end 193.675 91.059) (width 0.5) (layer B.Cu) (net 8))
 (segment (start 193.675 91.059) (end 197.231 91.059) (width 0.5) (layer B.Cu) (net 8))
 (segment (start 197.231 91.059) (end 197.48 90.81) (width 0.5) (layer B.Cu) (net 8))
 (segment (start 197.48 90.81) (end 197.48 89.125619) (width 0.5) (layer B.Cu) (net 8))
 (segment (start 207.137 95.631) (end 207.137 94.361) (width 0.5) (layer B.Cu) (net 9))
 (segment (start 208.915 92.583) (end 210.693 92.583) (width 0.5) (layer B.Cu) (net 9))
 (segment (start 207.137 94.361) (end 208.915 92.583) (width 0.5) (layer B.Cu) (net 9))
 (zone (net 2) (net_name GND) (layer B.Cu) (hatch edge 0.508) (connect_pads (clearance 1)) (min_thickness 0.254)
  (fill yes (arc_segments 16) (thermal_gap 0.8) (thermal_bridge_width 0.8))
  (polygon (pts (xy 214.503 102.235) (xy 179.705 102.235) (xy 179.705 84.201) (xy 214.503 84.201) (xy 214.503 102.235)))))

